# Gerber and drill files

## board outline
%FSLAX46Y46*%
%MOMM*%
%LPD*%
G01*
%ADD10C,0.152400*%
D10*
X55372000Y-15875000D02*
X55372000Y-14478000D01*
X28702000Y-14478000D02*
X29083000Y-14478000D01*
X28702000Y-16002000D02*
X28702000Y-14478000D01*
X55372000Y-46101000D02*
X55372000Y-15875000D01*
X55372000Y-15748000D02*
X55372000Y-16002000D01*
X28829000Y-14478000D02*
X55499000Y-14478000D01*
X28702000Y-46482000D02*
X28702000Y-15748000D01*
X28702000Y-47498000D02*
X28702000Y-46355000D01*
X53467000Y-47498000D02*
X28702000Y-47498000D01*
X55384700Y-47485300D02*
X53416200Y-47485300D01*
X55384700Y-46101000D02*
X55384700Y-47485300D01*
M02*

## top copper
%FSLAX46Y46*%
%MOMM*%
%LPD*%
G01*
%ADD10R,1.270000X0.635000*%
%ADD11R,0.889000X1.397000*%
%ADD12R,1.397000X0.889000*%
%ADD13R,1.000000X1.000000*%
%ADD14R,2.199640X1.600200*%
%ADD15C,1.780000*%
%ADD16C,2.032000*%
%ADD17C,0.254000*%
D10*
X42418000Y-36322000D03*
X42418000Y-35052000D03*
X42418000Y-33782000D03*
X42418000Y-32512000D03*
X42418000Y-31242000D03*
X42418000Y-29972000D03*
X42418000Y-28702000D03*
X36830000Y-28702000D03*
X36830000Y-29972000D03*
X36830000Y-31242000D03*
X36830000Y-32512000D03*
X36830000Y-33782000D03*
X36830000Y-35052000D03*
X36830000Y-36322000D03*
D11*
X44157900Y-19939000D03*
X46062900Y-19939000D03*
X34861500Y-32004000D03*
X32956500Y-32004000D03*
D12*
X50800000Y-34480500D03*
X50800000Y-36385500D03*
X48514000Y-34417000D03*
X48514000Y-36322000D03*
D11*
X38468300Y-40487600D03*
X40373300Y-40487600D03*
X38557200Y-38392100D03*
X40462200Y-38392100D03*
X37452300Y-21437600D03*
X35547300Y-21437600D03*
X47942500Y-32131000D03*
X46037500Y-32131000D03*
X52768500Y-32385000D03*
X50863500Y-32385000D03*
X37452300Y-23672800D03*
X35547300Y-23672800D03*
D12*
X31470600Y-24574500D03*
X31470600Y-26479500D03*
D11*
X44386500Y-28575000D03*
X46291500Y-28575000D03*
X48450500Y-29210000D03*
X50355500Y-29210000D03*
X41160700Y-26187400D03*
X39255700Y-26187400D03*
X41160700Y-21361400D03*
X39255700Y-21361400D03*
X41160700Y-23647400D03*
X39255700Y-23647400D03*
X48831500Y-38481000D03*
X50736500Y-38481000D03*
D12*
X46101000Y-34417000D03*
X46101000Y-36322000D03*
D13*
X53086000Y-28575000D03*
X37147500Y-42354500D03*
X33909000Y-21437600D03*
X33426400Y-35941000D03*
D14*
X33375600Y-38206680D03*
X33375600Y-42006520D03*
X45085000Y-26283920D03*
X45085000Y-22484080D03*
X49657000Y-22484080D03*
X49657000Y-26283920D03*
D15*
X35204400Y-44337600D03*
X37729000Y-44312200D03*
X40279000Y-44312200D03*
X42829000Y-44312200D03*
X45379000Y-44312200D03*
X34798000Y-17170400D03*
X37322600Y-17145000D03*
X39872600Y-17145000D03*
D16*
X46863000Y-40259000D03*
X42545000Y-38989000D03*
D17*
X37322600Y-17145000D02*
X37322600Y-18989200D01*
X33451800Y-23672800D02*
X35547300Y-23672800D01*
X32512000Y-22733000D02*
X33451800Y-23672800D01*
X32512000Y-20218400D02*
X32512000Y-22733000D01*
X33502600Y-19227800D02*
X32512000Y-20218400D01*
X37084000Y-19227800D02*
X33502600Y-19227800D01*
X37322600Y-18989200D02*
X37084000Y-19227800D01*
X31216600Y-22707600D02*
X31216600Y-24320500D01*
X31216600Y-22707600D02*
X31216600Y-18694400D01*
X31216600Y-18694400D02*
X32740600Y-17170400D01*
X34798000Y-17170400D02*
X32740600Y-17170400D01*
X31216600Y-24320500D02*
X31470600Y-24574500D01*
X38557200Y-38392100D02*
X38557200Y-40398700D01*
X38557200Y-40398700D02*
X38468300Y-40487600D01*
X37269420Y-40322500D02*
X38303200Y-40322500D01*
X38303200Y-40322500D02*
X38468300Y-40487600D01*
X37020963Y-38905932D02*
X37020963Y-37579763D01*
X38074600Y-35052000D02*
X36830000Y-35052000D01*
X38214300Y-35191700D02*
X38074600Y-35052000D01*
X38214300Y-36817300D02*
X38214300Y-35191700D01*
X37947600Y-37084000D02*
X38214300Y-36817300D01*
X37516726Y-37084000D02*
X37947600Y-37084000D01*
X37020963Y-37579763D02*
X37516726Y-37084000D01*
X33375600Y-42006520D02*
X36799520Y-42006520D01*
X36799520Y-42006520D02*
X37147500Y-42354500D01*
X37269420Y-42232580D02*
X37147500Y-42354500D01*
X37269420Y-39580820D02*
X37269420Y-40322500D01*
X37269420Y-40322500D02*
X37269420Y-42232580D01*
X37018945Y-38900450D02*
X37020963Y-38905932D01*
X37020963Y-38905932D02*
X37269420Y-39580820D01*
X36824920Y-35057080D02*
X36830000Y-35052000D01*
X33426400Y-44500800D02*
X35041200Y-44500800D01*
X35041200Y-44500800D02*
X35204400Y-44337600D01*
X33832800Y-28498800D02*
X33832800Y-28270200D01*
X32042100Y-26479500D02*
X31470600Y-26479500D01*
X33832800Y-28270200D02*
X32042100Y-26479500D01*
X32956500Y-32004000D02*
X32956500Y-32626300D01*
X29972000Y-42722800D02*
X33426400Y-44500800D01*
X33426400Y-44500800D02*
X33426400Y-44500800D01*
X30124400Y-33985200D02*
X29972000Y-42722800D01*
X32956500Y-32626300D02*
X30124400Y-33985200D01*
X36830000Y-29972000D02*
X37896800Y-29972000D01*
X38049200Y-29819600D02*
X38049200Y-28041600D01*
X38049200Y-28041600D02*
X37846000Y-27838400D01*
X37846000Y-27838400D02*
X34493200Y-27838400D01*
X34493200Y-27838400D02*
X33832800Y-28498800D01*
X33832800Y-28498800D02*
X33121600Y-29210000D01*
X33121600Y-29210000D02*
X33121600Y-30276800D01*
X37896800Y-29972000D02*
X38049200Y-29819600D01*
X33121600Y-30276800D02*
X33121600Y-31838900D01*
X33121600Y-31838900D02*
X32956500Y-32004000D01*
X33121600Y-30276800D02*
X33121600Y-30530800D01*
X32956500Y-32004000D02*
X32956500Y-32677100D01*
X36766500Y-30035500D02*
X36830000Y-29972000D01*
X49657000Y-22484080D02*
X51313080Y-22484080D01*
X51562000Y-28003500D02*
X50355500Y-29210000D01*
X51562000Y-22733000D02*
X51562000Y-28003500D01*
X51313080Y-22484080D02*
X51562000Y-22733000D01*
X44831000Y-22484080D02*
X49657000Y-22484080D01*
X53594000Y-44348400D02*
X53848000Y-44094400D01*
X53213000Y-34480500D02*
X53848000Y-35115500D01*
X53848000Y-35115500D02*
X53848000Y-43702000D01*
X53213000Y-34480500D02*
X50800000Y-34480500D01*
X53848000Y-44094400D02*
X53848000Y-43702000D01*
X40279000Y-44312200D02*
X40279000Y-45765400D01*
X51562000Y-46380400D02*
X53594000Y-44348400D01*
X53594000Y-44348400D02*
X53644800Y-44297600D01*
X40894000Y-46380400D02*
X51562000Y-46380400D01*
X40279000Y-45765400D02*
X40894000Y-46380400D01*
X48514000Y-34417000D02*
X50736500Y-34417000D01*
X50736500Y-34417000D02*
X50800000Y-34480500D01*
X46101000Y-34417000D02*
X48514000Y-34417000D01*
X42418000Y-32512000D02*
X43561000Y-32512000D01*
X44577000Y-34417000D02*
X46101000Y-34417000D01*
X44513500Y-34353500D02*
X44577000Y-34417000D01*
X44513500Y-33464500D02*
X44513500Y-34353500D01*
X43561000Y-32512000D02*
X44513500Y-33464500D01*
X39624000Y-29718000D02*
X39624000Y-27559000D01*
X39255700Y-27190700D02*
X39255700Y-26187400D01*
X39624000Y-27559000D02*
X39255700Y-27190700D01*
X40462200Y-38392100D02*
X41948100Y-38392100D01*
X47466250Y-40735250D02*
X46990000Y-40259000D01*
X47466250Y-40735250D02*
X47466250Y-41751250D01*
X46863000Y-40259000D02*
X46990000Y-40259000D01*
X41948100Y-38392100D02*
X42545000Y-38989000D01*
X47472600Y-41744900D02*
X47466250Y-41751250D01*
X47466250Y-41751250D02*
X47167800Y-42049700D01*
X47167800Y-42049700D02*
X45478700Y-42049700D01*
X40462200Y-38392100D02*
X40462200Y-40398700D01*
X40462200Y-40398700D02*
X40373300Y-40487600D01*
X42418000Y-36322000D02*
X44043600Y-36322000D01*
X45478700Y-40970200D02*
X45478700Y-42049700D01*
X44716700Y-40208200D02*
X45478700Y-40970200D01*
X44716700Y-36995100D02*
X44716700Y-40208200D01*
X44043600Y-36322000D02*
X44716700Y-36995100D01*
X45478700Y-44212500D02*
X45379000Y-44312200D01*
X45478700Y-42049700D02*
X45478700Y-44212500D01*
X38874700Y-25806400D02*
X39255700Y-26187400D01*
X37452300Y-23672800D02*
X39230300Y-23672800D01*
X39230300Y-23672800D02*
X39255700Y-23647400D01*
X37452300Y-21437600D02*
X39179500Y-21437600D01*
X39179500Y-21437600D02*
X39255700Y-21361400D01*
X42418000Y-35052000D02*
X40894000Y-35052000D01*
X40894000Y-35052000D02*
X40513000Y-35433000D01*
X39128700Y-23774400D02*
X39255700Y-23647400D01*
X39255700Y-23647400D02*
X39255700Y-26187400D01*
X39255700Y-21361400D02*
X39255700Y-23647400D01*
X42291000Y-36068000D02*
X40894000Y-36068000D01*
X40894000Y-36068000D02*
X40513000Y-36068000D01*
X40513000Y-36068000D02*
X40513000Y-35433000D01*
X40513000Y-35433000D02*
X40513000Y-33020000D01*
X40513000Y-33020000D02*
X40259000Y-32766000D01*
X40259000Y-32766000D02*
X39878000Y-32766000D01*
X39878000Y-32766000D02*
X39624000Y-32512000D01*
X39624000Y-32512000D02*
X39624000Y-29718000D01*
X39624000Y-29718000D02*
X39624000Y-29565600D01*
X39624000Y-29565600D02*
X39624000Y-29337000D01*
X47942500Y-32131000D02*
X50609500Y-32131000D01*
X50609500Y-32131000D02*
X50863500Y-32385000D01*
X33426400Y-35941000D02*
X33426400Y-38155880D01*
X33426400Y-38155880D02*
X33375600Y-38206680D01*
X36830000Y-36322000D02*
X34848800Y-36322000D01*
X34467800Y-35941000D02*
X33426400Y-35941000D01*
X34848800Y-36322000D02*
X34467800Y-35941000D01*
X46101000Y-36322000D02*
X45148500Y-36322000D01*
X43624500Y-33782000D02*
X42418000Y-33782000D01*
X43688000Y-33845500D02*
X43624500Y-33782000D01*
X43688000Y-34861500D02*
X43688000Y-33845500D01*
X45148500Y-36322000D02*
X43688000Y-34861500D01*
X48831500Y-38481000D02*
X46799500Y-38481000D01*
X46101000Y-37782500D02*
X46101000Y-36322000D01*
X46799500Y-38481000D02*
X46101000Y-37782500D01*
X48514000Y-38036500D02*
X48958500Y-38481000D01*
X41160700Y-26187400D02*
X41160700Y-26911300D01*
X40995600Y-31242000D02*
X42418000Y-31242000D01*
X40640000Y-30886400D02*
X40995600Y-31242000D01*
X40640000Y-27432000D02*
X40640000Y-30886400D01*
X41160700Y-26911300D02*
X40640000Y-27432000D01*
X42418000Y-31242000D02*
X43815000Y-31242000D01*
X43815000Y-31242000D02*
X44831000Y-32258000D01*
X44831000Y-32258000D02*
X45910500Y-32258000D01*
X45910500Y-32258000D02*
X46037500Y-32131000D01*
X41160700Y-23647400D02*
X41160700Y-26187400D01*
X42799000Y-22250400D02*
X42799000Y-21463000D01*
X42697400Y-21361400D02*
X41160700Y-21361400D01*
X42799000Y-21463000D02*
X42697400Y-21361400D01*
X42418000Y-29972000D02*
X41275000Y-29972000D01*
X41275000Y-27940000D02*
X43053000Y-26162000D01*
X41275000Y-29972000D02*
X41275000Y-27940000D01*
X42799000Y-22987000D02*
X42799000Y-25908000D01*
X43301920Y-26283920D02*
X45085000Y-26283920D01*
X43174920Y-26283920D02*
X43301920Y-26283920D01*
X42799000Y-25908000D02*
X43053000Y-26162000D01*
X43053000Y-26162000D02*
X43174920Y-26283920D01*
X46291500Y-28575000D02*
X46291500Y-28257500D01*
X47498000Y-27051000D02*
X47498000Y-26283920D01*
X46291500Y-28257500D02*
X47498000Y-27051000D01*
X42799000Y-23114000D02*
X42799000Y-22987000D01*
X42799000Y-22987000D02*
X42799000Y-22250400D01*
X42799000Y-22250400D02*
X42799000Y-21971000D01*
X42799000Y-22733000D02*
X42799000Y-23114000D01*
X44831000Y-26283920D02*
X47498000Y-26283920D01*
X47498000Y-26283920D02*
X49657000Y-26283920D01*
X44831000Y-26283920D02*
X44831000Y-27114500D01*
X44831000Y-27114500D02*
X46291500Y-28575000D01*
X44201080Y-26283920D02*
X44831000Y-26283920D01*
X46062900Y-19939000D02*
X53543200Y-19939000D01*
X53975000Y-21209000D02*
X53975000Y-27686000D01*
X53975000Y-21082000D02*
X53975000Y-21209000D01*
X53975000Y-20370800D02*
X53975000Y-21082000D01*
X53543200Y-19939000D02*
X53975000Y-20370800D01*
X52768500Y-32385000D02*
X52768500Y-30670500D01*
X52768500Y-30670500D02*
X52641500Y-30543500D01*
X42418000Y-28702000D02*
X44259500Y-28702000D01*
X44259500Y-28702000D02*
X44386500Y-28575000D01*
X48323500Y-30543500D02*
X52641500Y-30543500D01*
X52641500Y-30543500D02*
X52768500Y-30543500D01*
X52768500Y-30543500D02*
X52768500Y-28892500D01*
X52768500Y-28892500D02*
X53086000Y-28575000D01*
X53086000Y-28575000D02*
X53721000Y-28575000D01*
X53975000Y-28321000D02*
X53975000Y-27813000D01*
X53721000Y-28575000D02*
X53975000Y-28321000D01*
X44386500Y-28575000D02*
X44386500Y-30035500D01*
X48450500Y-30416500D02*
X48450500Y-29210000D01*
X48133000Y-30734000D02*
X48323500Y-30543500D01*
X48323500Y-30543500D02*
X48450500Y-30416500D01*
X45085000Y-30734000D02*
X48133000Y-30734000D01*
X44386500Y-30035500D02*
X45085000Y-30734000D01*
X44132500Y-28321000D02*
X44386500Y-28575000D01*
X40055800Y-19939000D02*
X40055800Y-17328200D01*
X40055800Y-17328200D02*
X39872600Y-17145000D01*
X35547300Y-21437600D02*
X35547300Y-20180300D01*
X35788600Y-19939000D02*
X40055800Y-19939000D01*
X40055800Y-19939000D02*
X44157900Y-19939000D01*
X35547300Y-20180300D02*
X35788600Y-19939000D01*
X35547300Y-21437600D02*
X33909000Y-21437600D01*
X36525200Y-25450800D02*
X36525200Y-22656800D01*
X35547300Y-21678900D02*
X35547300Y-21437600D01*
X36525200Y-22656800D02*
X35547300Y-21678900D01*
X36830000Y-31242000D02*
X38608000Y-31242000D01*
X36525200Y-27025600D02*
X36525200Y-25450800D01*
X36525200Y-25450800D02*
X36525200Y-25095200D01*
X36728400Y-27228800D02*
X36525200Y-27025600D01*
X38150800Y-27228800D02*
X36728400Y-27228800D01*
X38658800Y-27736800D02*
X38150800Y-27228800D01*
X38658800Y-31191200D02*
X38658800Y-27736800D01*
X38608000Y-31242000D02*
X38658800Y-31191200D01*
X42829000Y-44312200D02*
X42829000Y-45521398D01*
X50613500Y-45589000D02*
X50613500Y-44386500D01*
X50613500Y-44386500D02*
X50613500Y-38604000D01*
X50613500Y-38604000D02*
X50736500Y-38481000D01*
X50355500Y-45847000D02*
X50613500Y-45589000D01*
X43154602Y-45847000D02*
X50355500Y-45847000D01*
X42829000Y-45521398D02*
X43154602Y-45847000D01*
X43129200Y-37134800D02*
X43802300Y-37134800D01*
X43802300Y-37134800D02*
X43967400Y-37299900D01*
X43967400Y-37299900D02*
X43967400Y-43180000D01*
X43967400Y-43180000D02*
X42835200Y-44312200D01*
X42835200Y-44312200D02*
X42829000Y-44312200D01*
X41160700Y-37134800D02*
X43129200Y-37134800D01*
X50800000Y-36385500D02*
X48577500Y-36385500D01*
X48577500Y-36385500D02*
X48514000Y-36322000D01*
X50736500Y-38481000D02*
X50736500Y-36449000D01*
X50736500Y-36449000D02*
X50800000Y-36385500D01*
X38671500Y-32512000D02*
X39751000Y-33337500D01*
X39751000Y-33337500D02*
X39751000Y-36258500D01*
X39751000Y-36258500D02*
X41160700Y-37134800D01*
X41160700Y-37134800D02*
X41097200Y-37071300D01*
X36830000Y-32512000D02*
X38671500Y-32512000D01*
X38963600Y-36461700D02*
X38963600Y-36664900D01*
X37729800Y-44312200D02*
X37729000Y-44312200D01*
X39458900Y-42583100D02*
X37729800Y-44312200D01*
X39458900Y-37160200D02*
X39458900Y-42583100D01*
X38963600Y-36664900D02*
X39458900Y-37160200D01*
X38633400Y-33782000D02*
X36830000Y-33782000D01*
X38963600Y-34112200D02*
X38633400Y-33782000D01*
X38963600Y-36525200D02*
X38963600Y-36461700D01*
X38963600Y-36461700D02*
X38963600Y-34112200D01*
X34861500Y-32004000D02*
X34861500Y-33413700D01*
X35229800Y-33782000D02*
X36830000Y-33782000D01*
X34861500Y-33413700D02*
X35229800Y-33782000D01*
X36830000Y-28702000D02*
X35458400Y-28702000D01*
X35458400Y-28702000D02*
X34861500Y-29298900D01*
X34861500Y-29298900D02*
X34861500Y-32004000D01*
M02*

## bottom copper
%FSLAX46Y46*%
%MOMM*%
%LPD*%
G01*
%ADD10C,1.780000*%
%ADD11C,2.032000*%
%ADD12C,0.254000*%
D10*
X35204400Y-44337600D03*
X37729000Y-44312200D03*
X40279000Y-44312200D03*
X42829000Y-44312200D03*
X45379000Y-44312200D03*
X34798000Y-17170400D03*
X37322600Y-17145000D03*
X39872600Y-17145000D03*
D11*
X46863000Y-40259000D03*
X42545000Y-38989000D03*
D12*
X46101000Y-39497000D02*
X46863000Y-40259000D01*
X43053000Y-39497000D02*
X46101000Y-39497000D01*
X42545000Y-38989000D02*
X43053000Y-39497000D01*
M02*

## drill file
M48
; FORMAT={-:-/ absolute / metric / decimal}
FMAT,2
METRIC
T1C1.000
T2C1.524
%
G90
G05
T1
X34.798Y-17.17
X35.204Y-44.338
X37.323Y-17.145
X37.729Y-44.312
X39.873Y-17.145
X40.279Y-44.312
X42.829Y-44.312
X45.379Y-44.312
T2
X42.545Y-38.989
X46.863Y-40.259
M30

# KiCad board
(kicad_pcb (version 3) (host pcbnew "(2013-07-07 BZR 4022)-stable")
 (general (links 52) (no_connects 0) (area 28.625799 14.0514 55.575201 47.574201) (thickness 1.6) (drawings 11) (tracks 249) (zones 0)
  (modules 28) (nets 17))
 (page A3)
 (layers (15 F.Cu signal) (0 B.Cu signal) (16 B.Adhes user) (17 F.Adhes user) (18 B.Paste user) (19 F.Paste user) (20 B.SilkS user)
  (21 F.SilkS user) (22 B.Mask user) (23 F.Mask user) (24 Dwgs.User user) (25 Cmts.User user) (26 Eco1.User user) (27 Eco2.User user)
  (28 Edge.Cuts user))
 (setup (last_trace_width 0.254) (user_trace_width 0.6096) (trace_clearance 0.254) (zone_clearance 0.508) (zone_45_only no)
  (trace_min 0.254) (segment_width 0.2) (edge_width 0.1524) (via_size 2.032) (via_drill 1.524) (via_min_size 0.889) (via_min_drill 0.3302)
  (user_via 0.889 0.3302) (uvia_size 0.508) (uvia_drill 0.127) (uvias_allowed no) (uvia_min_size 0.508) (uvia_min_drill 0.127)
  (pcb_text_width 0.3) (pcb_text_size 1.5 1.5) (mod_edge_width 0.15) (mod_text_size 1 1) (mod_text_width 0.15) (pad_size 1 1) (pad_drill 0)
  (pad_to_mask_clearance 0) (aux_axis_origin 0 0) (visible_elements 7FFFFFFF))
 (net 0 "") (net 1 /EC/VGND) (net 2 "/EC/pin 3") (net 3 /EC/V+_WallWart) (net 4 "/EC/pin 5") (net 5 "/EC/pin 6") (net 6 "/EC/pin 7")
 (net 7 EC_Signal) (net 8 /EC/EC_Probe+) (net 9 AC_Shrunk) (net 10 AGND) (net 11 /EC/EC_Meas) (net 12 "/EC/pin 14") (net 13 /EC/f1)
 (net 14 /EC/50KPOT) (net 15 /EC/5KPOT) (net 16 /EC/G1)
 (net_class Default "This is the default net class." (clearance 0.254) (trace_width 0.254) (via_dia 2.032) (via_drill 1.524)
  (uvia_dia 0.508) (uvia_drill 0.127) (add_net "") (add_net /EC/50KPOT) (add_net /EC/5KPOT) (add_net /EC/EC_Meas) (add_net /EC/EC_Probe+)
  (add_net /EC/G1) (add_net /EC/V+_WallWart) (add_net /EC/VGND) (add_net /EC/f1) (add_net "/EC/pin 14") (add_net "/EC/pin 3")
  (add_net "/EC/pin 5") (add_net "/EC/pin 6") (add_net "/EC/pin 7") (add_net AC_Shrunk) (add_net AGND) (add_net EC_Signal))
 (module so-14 (layer F.Cu) (at 39.624 32.512 90)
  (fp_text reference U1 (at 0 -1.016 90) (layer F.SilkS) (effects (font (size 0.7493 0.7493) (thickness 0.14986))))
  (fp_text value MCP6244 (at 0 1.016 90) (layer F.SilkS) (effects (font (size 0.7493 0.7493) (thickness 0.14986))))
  (pad 1 smd rect (at -3.81 2.794 90) (size 0.635 1.27) (layers F.Cu F.Paste F.Mask) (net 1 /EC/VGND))
  (pad 2 smd rect (at -2.54 2.794 90) (size 0.635 1.27) (layers F.Cu F.Paste F.Mask) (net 1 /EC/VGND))
  (pad 3 smd rect (at -1.27 2.794 90) (size 0.635 1.27) (layers F.Cu F.Paste F.Mask) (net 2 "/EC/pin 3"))
  (pad 4 smd rect (at 0 2.794 90) (size 0.635 1.27) (layers F.Cu F.Paste F.Mask) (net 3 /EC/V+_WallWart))
  (pad 5 smd rect (at 1.27 2.794 90) (size 0.635 1.27) (layers F.Cu F.Paste F.Mask) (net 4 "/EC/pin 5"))
  (pad 6 smd rect (at 2.54 2.794 90) (size 0.635 1.27) (layers F.Cu F.Paste F.Mask) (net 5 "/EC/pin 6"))
  (pad 7 smd rect (at 3.81 2.794 90) (size 0.635 1.27) (layers F.Cu F.Paste F.Mask) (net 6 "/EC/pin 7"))
  (pad 8 smd rect (at 3.81 -2.794 90) (size 0.635 1.27) (layers F.Cu F.Paste F.Mask) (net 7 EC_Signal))
  (pad 9 smd rect (at 2.54 -2.794 90) (size 0.635 1.27) (layers F.Cu F.Paste F.Mask) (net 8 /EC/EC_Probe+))
  (pad 10 smd rect (at 1.27 -2.794 90) (size 0.635 1.27) (layers F.Cu F.Paste F.Mask) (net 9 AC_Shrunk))
  (pad 11 smd rect (at 0 -2.794 90) (size 0.635 1.27) (layers F.Cu F.Paste F.Mask) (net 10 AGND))
  (pad 12 smd rect (at -1.27 -2.794 90) (size 0.635 1.27) (layers F.Cu F.Paste F.Mask) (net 7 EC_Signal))
  (pad 13 smd rect (at -2.54 -2.794 90) (size 0.635 1.27) (layers F.Cu F.Paste F.Mask) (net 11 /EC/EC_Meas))
  (pad 14 smd rect (at -3.81 -2.794 90) (size 0.635 1.27) (layers F.Cu F.Paste F.Mask) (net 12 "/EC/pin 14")))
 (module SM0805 (layer F.Cu) (at 45.1104 19.939)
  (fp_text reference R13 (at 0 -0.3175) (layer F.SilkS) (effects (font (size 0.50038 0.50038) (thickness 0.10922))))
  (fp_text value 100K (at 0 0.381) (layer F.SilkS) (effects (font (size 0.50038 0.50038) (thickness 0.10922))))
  (pad 1 smd rect (at -0.9525 0) (size 0.889 1.397) (layers F.Cu F.Paste F.Mask) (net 9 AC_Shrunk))
  (pad 2 smd rect (at 0.9525 0) (size 0.889 1.397) (layers F.Cu F.Paste F.Mask) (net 6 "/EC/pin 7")))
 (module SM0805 (layer F.Cu) (at 33.909 32.004 180)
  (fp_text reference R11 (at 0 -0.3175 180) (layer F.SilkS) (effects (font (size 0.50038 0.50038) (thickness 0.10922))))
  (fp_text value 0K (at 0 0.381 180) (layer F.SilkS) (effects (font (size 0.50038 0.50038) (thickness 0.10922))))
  (pad 1 smd rect (at -0.9525 0 180) (size 0.889 1.397) (layers F.Cu F.Paste F.Mask) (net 7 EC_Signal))
  (pad 2 smd rect (at 0.9525 0 180) (size 0.889 1.397) (layers F.Cu F.Paste F.Mask) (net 8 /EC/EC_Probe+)))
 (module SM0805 (layer F.Cu) (at 50.8 35.433 270)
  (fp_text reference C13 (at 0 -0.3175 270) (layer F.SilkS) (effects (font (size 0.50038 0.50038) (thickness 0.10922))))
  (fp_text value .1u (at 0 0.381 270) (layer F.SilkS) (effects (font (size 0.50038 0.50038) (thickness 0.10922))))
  (pad 1 smd rect (at -0.9525 0 270) (size 0.889 1.397) (layers F.Cu F.Paste F.Mask) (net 3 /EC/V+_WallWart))
  (pad 2 smd rect (at 0.9525 0 270) (size 0.889 1.397) (layers F.Cu F.Paste F.Mask) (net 10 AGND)))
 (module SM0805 (layer F.Cu) (at 48.514 35.3695 270)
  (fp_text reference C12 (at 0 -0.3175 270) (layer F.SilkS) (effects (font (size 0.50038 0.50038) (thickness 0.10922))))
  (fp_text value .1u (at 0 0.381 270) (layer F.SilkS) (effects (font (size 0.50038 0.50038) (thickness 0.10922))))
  (pad 1 smd rect (at -0.9525 0 270) (size 0.889 1.397) (layers F.Cu F.Paste F.Mask) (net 3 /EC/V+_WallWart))
  (pad 2 smd rect (at 0.9525 0 270) (size 0.889 1.397) (layers F.Cu F.Paste F.Mask) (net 10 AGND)))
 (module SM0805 (layer F.Cu) (at 39.4208 40.4876)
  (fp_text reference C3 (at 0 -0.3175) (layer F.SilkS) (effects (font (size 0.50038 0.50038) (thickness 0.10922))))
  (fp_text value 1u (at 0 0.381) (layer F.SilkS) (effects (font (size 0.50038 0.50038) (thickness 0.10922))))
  (pad 1 smd rect (at -0.9525 0) (size 0.889 1.397) (layers F.Cu F.Paste F.Mask) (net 11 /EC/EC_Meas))
  (pad 2 smd rect (at 0.9525 0) (size 0.889 1.397) (layers F.Cu F.Paste F.Mask) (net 1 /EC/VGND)))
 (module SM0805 (layer F.Cu) (at 39.5097 38.3921)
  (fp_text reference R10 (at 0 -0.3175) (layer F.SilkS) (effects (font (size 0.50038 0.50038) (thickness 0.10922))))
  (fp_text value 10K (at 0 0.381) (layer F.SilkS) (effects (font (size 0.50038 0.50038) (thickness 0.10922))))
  (pad 1 smd rect (at -0.9525 0) (size 0.889 1.397) (layers F.Cu F.Paste F.Mask) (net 11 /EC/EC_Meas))
  (pad 2 smd rect (at 0.9525 0) (size 0.889 1.397) (layers F.Cu F.Paste F.Mask) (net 1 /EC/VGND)))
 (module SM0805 (layer F.Cu) (at 36.4998 21.4376 180)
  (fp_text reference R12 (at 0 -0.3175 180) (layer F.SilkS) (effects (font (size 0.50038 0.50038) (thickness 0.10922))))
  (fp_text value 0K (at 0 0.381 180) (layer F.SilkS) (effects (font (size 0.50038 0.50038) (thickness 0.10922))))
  (pad 1 smd rect (at -0.9525 0 180) (size 0.889 1.397) (layers F.Cu F.Paste F.Mask) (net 1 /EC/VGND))
  (pad 2 smd rect (at 0.9525 0 180) (size 0.889 1.397) (layers F.Cu F.Paste F.Mask) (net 9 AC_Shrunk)))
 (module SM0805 (layer F.Cu) (at 46.99 32.131 180)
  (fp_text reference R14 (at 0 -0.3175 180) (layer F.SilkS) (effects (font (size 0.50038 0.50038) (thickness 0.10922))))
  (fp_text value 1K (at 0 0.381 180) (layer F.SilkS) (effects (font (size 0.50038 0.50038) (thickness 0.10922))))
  (pad 1 smd rect (at -0.9525 0 180) (size 0.889 1.397) (layers F.Cu F.Paste F.Mask) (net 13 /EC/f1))
  (pad 2 smd rect (at 0.9525 0 180) (size 0.889 1.397) (layers F.Cu F.Paste F.Mask) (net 4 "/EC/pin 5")))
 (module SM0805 (layer F.Cu) (at 51.816 32.385 180)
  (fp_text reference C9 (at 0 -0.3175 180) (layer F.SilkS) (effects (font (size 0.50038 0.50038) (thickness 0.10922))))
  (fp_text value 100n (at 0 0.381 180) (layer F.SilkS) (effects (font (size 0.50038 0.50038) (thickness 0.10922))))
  (pad 1 smd rect (at -0.9525 0 180) (size 0.889 1.397) (layers F.Cu F.Paste F.Mask) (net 6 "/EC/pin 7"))
  (pad 2 smd rect (at 0.9525 0 180) (size 0.889 1.397) (layers F.Cu F.Paste F.Mask) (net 13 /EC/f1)))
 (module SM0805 (layer F.Cu) (at 36.4998 23.6728 180)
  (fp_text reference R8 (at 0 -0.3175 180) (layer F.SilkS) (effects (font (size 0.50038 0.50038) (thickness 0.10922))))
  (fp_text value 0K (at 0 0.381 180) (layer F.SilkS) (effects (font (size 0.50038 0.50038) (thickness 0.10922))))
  (pad 1 smd rect (at -0.9525 0 180) (size 0.889 1.397) (layers F.Cu F.Paste F.Mask) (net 1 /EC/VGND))
  (pad 2 smd rect (at 0.9525 0 180) (size 0.889 1.397) (layers F.Cu F.Paste F.Mask) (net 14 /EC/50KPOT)))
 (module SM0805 (layer F.Cu) (at 31.4706 25.527 270)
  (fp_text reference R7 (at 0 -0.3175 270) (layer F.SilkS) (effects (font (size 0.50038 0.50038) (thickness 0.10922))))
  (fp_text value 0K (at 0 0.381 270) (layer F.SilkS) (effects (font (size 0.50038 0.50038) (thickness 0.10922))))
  (pad 1 smd rect (at -0.9525 0 270) (size 0.889 1.397) (layers F.Cu F.Paste F.Mask) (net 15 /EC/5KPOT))
  (pad 2 smd rect (at 0.9525 0 270) (size 0.889 1.397) (layers F.Cu F.Paste F.Mask) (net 8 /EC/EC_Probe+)))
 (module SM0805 (layer F.Cu) (at 45.339 28.575)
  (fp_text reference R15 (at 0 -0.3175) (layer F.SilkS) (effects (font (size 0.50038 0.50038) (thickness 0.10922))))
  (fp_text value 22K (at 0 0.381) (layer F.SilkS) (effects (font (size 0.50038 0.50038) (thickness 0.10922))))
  (pad 1 smd rect (at -0.9525 0) (size 0.889 1.397) (layers F.Cu F.Paste F.Mask) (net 6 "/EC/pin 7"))
  (pad 2 smd rect (at 0.9525 0) (size 0.889 1.397) (layers F.Cu F.Paste F.Mask) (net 5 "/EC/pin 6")))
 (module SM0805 (layer F.Cu) (at 49.403 29.21)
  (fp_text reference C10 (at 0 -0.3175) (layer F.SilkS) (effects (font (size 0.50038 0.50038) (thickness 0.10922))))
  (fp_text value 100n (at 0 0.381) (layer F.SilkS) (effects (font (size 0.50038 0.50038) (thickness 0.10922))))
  (pad 1 smd rect (at -0.9525 0) (size 0.889 1.397) (layers F.Cu F.Paste F.Mask) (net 6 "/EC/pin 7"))
  (pad 2 smd rect (at 0.9525 0) (size 0.889 1.397) (layers F.Cu F.Paste F.Mask) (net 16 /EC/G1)))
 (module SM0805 (layer F.Cu) (at 40.2082 26.1874 180)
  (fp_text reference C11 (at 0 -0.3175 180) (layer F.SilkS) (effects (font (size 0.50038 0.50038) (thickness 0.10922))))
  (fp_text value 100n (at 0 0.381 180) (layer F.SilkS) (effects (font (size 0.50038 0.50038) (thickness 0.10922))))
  (pad 1 smd rect (at -0.9525 0 180) (size 0.889 1.397) (layers F.Cu F.Paste F.Mask) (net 4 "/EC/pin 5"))
  (pad 2 smd rect (at 0.9525 0 180) (size 0.889 1.397) (layers F.Cu F.Paste F.Mask) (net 1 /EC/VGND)))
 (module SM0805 (layer F.Cu) (at 40.2082 21.3614 180)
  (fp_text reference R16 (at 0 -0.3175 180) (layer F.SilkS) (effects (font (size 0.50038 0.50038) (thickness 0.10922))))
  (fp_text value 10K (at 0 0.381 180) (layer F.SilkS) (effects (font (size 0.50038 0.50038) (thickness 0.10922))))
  (pad 1 smd rect (at -0.9525 0 180) (size 0.889 1.397) (layers F.Cu F.Paste F.Mask) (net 5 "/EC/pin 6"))
  (pad 2 smd rect (at 0.9525 0 180) (size 0.889 1.397) (layers F.Cu F.Paste F.Mask) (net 1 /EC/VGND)))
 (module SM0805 (layer F.Cu) (at 40.2082 23.6474 180)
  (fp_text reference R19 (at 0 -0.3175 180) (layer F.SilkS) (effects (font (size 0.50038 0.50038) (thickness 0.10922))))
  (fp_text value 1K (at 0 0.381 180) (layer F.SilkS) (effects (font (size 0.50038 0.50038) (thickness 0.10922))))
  (pad 1 smd rect (at -0.9525 0 180) (size 0.889 1.397) (layers F.Cu F.Paste F.Mask) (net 4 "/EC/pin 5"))
  (pad 2 smd rect (at 0.9525 0 180) (size 0.889 1.397) (layers F.Cu F.Paste F.Mask) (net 1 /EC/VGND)))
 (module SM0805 (layer F.Cu) (at 49.784 38.481)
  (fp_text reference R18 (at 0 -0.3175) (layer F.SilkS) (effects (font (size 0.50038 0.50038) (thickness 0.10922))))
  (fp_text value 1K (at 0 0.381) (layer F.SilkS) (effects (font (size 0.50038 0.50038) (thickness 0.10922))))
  (pad 1 smd rect (at -0.9525 0) (size 0.889 1.397) (layers F.Cu F.Paste F.Mask) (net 2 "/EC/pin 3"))
  (pad 2 smd rect (at 0.9525 0) (size 0.889 1.397) (layers F.Cu F.Paste F.Mask) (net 10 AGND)))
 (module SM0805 (layer F.Cu) (at 46.101 35.3695 270)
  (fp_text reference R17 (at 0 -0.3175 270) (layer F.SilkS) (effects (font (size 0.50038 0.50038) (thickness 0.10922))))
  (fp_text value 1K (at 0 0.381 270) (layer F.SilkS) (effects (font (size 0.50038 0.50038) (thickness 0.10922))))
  (pad 1 smd rect (at -0.9525 0 270) (size 0.889 1.397) (layers F.Cu F.Paste F.Mask) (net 3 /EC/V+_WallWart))
  (pad 2 smd rect (at 0.9525 0 270) (size 0.889 1.397) (layers F.Cu F.Paste F.Mask) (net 2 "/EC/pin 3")))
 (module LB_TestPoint (layer F.Cu) (at 53.086 28.575)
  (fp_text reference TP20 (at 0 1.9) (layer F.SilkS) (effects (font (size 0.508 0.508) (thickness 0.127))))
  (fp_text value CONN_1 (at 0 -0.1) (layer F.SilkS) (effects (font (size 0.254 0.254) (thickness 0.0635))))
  (pad 1 smd rect (at 0 0) (size 1 1) (layers F.Cu F.Paste F.Mask) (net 6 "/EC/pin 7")))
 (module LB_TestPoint (layer F.Cu) (at 37.1475 42.3545 90)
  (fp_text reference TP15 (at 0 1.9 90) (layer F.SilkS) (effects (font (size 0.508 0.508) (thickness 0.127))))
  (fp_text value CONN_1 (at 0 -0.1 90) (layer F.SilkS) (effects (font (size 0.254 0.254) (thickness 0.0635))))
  (pad 1 smd rect (at 0 0 90) (size 1 1) (layers F.Cu F.Paste F.Mask) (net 11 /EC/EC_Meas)))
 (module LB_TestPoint (layer F.Cu) (at 33.909 21.4376)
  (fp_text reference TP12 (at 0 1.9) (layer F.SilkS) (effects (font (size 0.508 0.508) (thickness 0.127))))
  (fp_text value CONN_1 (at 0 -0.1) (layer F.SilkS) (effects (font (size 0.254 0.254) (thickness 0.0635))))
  (pad 1 smd rect (at 0 0) (size 1 1) (layers F.Cu F.Paste F.Mask) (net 9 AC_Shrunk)))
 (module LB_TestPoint (layer F.Cu) (at 33.4264 35.941)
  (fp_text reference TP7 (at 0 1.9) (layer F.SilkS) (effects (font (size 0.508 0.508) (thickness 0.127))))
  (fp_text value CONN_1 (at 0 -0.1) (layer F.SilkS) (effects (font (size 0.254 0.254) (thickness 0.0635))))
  (pad 1 smd rect (at 0 0) (size 1 1) (layers F.Cu F.Paste F.Mask) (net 12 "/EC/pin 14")))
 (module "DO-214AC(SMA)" (layer F.Cu) (at 33.3756 40.1066 270)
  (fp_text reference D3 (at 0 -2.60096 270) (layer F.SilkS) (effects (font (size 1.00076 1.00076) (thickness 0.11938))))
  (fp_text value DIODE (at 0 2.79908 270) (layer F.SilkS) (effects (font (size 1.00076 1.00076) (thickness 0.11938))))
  (pad 1 smd rect (at -1.89992 0 270) (size 1.6002 2.19964) (layers F.Cu F.Paste F.Mask) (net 12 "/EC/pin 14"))
  (pad 2 smd rect (at 1.89992 0 270) (size 1.6002 2.19964) (layers F.Cu F.Paste F.Mask) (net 11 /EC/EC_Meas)))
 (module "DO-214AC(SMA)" (layer F.Cu) (at 45.085 24.384 90)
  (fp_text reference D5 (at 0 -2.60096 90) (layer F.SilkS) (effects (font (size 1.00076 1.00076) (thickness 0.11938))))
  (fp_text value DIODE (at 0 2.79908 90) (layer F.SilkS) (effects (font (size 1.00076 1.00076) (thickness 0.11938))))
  (pad 1 smd rect (at -1.89992 0 90) (size 1.6002 2.19964) (layers F.Cu F.Paste F.Mask) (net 5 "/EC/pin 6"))
  (pad 2 smd rect (at 1.89992 0 90) (size 1.6002 2.19964) (layers F.Cu F.Paste F.Mask) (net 16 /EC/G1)))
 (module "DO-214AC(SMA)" (layer F.Cu) (at 49.657 24.384 270)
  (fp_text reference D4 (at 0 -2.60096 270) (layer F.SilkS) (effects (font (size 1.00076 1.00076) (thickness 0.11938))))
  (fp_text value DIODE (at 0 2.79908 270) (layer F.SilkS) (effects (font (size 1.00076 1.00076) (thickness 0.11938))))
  (pad 1 smd rect (at -1.89992 0 270) (size 1.6002 2.19964) (layers F.Cu F.Paste F.Mask) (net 16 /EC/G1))
  (pad 2 smd rect (at 1.89992 0 270) (size 1.6002 2.19964) (layers F.Cu F.Paste F.Mask) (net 5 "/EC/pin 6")))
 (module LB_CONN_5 (layer F.Cu) (at 35.2044 44.2976)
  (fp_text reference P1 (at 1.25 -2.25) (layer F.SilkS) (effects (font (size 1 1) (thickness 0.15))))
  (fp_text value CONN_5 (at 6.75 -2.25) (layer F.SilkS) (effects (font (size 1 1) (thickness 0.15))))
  (pad 1 thru_hole circle (at 0 0.04) (size 1.78 1.78) (drill 1) (layers *.Cu *.Mask F.SilkS) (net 8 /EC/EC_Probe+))
  (pad 2 thru_hole circle (at 2.5246 0.0146) (size 1.78 1.78) (drill 1) (layers *.Cu *.Mask F.SilkS) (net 7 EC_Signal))
  (pad 3 thru_hole circle (at 5.0746 0.0146) (size 1.78 1.78) (drill 1) (layers *.Cu *.Mask F.SilkS) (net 3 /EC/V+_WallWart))
  (pad 4 thru_hole circle (at 7.6246 0.0146) (size 1.78 1.78) (drill 1) (layers *.Cu *.Mask F.SilkS) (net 10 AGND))
  (pad 5 thru_hole circle (at 10.1746 0.0146) (size 1.78 1.78) (drill 1) (layers *.Cu *.Mask F.SilkS) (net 1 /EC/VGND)))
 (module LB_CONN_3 (layer F.Cu) (at 34.798 14.6304)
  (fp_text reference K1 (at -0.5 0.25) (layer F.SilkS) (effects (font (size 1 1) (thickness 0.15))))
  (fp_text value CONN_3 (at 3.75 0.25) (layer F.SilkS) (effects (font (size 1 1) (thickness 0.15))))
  (pad 1 thru_hole circle (at 0 2.54) (size 1.78 1.78) (drill 1) (layers *.Cu *.Mask F.SilkS) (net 15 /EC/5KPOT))
  (pad 2 thru_hole circle (at 2.5246 2.5146) (size 1.78 1.78) (drill 1) (layers *.Cu *.Mask F.SilkS) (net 14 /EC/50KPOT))
  (pad 3 thru_hole circle (at 5.0746 2.5146) (size 1.78 1.78) (drill 1) (layers *.Cu *.Mask F.SilkS) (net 9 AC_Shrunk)))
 (gr_line (start 55.372 15.875) (end 55.372 14.478) (angle 90) (layer Edge.Cuts) (width 0.1524))
 (gr_line (start 28.702 14.478) (end 29.083 14.478) (angle 90) (layer Edge.Cuts) (width 0.1524))
 (gr_line (start 28.702 16.002) (end 28.702 14.478) (angle 90) (layer Edge.Cuts) (width 0.1524))
 (gr_line (start 55.372 46.101) (end 55.372 15.875) (angle 90) (layer Edge.Cuts) (width 0.1524))
 (gr_line (start 55.372 15.748) (end 55.372 16.002) (angle 90) (layer Edge.Cuts) (width 0.1524))
 (gr_line (start 28.829 14.478) (end 55.499 14.478) (angle 90) (layer Edge.Cuts) (width 0.1524))
 (gr_line (start 28.702 46.482) (end 28.702 15.748) (angle 90) (layer Edge.Cuts) (width 0.1524))
 (gr_line (start 28.702 47.498) (end 28.702 46.355) (angle 90) (layer Edge.Cuts) (width 0.1524))
 (gr_line (start 53.467 47.498) (end 28.702 47.498) (angle 90) (layer Edge.Cuts) (width 0.1524))
 (gr_line (start 55.3847 47.4853) (end 53.4162 47.4853) (angle 90) (layer Edge.Cuts) (width 0.1524))
 (gr_line (start 55.3847 46.101) (end 55.3847 47.4853) (angle 90) (layer Edge.Cuts) (width 0.1524))
 (segment (start 37.3226 17.145) (end 37.3226 18.9892) (width 0.254) (layer F.Cu) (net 14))
 (segment (start 33.4518 23.6728) (end 35.5473 23.6728) (width 0.254) (layer F.Cu) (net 14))
 (segment (start 32.512 22.733) (end 33.4518 23.6728) (width 0.254) (layer F.Cu) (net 14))
 (segment (start 32.512 20.2184) (end 32.512 22.733) (width 0.254) (layer F.Cu) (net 14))
 (segment (start 33.5026 19.2278) (end 32.512 20.2184) (width 0.254) (layer F.Cu) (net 14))
 (segment (start 37.084 19.2278) (end 33.5026 19.2278) (width 0.254) (layer F.Cu) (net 14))
 (segment (start 37.3226 18.9892) (end 37.084 19.2278) (width 0.254) (layer F.Cu) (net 14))
 (segment (start 31.2166 22.7076) (end 31.2166 24.3205) (width 0.254) (layer F.Cu) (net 15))
 (segment (start 31.2166 22.7076) (end 31.2166 18.6944) (width 0.254) (layer F.Cu) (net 15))
 (segment (start 31.2166 18.6944) (end 32.7406 17.1704) (width 0.254) (layer F.Cu) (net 15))
 (segment (start 34.798 17.1704) (end 32.7406 17.1704) (width 0.254) (layer F.Cu) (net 15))
 (segment (start 31.2166 24.3205) (end 31.4706 24.5745) (width 0.254) (layer F.Cu) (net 15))
 (segment (start 38.5572 38.3921) (end 38.5572 40.3987) (width 0.254) (layer F.Cu) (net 11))
 (segment (start 38.5572 40.3987) (end 38.4683 40.4876) (width 0.254) (layer F.Cu) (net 11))
 (segment (start 37.26942 40.3225) (end 38.3032 40.3225) (width 0.254) (layer F.Cu) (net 11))
 (segment (start 38.3032 40.3225) (end 38.4683 40.4876) (width 0.254) (layer F.Cu) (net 11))
 (segment (start 37.020963 38.905932) (end 37.020963 37.579763) (width 0.254) (layer F.Cu) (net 11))
 (segment (start 38.0746 35.052) (end 36.83 35.052) (width 0.254) (layer F.Cu) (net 11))
 (segment (start 38.2143 35.1917) (end 38.0746 35.052) (width 0.254) (layer F.Cu) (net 11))
 (segment (start 38.2143 36.8173) (end 38.2143 35.1917) (width 0.254) (layer F.Cu) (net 11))
 (segment (start 37.9476 37.084) (end 38.2143 36.8173) (width 0.254) (layer F.Cu) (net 11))
 (segment (start 37.516726 37.084) (end 37.9476 37.084) (width 0.254) (layer F.Cu) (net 11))
 (segment (start 37.020963 37.579763) (end 37.516726 37.084) (width 0.254) (layer F.Cu) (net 11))
 (segment (start 33.3756 42.00652) (end 36.79952 42.00652) (width 0.254) (layer F.Cu) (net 11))
 (segment (start 36.79952 42.00652) (end 37.1475 42.3545) (width 0.254) (layer F.Cu) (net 11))
 (segment (start 37.26942 42.23258) (end 37.1475 42.3545) (width 0.254) (layer F.Cu) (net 11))
 (segment (start 37.26942 39.58082) (end 37.26942 40.3225) (width 0.254) (layer F.Cu) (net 11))
 (segment (start 37.26942 40.3225) (end 37.26942 42.23258) (width 0.254) (layer F.Cu) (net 11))
 (segment (start 37.018945 38.90045) (end 37.020963 38.905932) (width 0.254) (layer F.Cu) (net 11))
 (segment (start 37.020963 38.905932) (end 37.26942 39.58082) (width 0.254) (layer F.Cu) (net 11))
 (segment (start 36.82492 35.05708) (end 36.83 35.052) (width 0.254) (layer F.Cu) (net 11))
 (segment (start 33.4264 44.5008) (end 35.0412 44.5008) (width 0.254) (layer F.Cu) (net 8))
 (segment (start 35.0412 44.5008) (end 35.2044 44.3376) (width 0.254) (layer F.Cu) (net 8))
 (segment (start 33.8328 28.4988) (end 33.8328 28.2702) (width 0.254) (layer F.Cu) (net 8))
 (segment (start 32.0421 26.4795) (end 31.4706 26.4795) (width 0.254) (layer F.Cu) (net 8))
 (segment (start 33.8328 28.2702) (end 32.0421 26.4795) (width 0.254) (layer F.Cu) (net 8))
 (segment (start 32.9565 32.004) (end 32.9565 32.6263) (width 0.254) (layer F.Cu) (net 8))
 (segment (start 29.972 42.7228) (end 33.4264 44.5008) (width 0.254) (layer F.Cu) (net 8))
 (segment (start 33.4264 44.5008) (end 33.4264 44.5008) (width 0.254) (layer F.Cu) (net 8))
 (segment (start 30.1244 33.9852) (end 29.972 42.7228) (width 0.254) (layer F.Cu) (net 8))
 (segment (start 32.9565 32.6263) (end 30.1244 33.9852) (width 0.254) (layer F.Cu) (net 8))
 (segment (start 36.83 29.972) (end 37.8968 29.972) (width 0.254) (layer F.Cu) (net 8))
 (segment (start 38.0492 29.8196) (end 38.0492 28.0416) (width 0.254) (layer F.Cu) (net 8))
 (segment (start 38.0492 28.0416) (end 37.846 27.8384) (width 0.254) (layer F.Cu) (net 8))
 (segment (start 37.846 27.8384) (end 34.4932 27.8384) (width 0.254) (layer F.Cu) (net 8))
 (segment (start 34.4932 27.8384) (end 33.8328 28.4988) (width 0.254) (layer F.Cu) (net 8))
 (segment (start 33.8328 28.4988) (end 33.1216 29.21) (width 0.254) (layer F.Cu) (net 8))
 (segment (start 33.1216 29.21) (end 33.1216 30.2768) (width 0.254) (layer F.Cu) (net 8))
 (segment (start 37.8968 29.972) (end 38.0492 29.8196) (width 0.254) (layer F.Cu) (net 8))
 (segment (start 33.1216 30.2768) (end 33.1216 31.8389) (width 0.254) (layer F.Cu) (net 8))
 (segment (start 33.1216 31.8389) (end 32.9565 32.004) (width 0.254) (layer F.Cu) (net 8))
 (segment (start 33.1216 30.2768) (end 33.1216 30.5308) (width 0.254) (layer F.Cu) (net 8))
 (segment (start 32.9565 32.004) (end 32.9565 32.6771) (width 0.254) (layer F.Cu) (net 8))
 (segment (start 36.7665 30.0355) (end 36.83 29.972) (width 0.254) (layer F.Cu) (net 8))
 (segment (start 49.657 22.48408) (end 51.31308 22.48408) (width 0.254) (layer F.Cu) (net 16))
 (segment (start 51.562 28.0035) (end 50.3555 29.21) (width 0.254) (layer F.Cu) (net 16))
 (segment (start 51.562 22.733) (end 51.562 28.0035) (width 0.254) (layer F.Cu) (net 16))
 (segment (start 51.31308 22.48408) (end 51.562 22.733) (width 0.254) (layer F.Cu) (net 16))
 (segment (start 44.831 22.48408) (end 49.657 22.48408) (width 0.254) (layer F.Cu) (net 16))
 (segment (start 53.594 44.3484) (end 53.848 44.0944) (width 0.254) (layer F.Cu) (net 3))
 (segment (start 53.213 34.4805) (end 53.848 35.1155) (width 0.254) (layer F.Cu) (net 3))
 (segment (start 53.848 35.1155) (end 53.848 43.702) (width 0.254) (layer F.Cu) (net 3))
 (segment (start 53.213 34.4805) (end 50.8 34.4805) (width 0.254) (layer F.Cu) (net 3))
 (segment (start 53.848 44.0944) (end 53.848 43.702) (width 0.254) (layer F.Cu) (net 3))
 (segment (start 40.279 44.3122) (end 40.279 45.7654) (width 0.254) (layer F.Cu) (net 3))
 (segment (start 51.562 46.3804) (end 53.594 44.3484) (width 0.254) (layer F.Cu) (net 3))
 (segment (start 53.594 44.3484) (end 53.6448 44.2976) (width 0.254) (layer F.Cu) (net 3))
 (segment (start 40.894 46.3804) (end 51.562 46.3804) (width 0.254) (layer F.Cu) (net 3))
 (segment (start 40.279 45.7654) (end 40.894 46.3804) (width 0.254) (layer F.Cu) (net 3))
 (segment (start 48.514 34.417) (end 50.7365 34.417) (width 0.254) (layer F.Cu) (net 3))
 (segment (start 50.7365 34.417) (end 50.8 34.4805) (width 0.254) (layer F.Cu) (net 3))
 (segment (start 46.101 34.417) (end 48.514 34.417) (width 0.254) (layer F.Cu) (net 3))
 (segment (start 42.418 32.512) (end 43.561 32.512) (width 0.254) (layer F.Cu) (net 3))
 (segment (start 44.577 34.417) (end 46.101 34.417) (width 0.254) (layer F.Cu) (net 3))
 (segment (start 44.5135 34.3535) (end 44.577 34.417) (width 0.254) (layer F.Cu) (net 3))
 (segment (start 44.5135 33.4645) (end 44.5135 34.3535) (width 0.254) (layer F.Cu) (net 3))
 (segment (start 43.561 32.512) (end 44.5135 33.4645) (width 0.254) (layer F.Cu) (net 3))
 (segment (start 39.624 29.718) (end 39.624 27.559) (width 0.254) (layer F.Cu) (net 1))
 (segment (start 39.2557 27.1907) (end 39.2557 26.1874) (width 0.254) (layer F.Cu) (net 1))
 (segment (start 39.624 27.559) (end 39.2557 27.1907) (width 0.254) (layer F.Cu) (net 1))
 (segment (start 40.4622 38.3921) (end 41.9481 38.3921) (width 0.254) (layer F.Cu) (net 1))
 (segment (start 47.46625 40.73525) (end 46.99 40.259) (width 0.254) (layer F.Cu) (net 1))
 (segment (start 47.46625 40.73525) (end 47.46625 41.75125) (width 0.254) (layer F.Cu) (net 1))
 (segment (start 46.863 40.259) (end 46.99 40.259) (width 0.254) (layer F.Cu) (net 1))
 (via (at 46.863 40.259) (size 2.032) (layers F.Cu B.Cu) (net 1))
 (segment (start 46.101 39.497) (end 46.863 40.259) (width 0.254) (layer B.Cu) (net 1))
 (segment (start 43.053 39.497) (end 46.101 39.497) (width 0.254) (layer B.Cu) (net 1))
 (segment (start 42.545 38.989) (end 43.053 39.497) (width 0.254) (layer B.Cu) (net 1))
 (via (at 42.545 38.989) (size 2.032) (layers F.Cu B.Cu) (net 1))
 (segment (start 41.9481 38.3921) (end 42.545 38.989) (width 0.254) (layer F.Cu) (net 1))
 (segment (start 47.4726 41.7449) (end 47.46625 41.75125) (width 0.254) (layer F.Cu) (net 1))
 (segment (start 47.46625 41.75125) (end 47.1678 42.0497) (width 0.254) (layer F.Cu) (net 1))
 (segment (start 47.1678 42.0497) (end 45.4787 42.0497) (width 0.254) (layer F.Cu) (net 1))
 (segment (start 40.4622 38.3921) (end 40.4622 40.3987) (width 0.254) (layer F.Cu) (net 1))
 (segment (start 40.4622 40.3987) (end 40.3733 40.4876) (width 0.254) (layer F.Cu) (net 1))
 (segment (start 42.418 36.322) (end 44.0436 36.322) (width 0.254) (layer F.Cu) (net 1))
 (segment (start 45.4787 40.9702) (end 45.4787 42.0497) (width 0.254) (layer F.Cu) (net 1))
 (segment (start 44.7167 40.2082) (end 45.4787 40.9702) (width 0.254) (layer F.Cu) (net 1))
 (segment (start 44.7167 36.9951) (end 44.7167 40.2082) (width 0.254) (layer F.Cu) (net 1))
 (segment (start 44.0436 36.322) (end 44.7167 36.9951) (width 0.254) (layer F.Cu) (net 1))
 (segment (start 45.4787 44.2125) (end 45.379 44.3122) (width 0.254) (layer F.Cu) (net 1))
 (segment (start 45.4787 42.0497) (end 45.4787 44.2125) (width 0.254) (layer F.Cu) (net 1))
 (segment (start 38.8747 25.8064) (end 39.2557 26.1874) (width 0.254) (layer F.Cu) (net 1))
 (segment (start 37.4523 23.6728) (end 39.2303 23.6728) (width 0.254) (layer F.Cu) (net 1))
 (segment (start 39.2303 23.6728) (end 39.2557 23.6474) (width 0.254) (layer F.Cu) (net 1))
 (segment (start 37.4523 21.4376) (end 39.1795 21.4376) (width 0.254) (layer F.Cu) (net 1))
 (segment (start 39.1795 21.4376) (end 39.2557 21.3614) (width 0.254) (layer F.Cu) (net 1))
 (segment (start 42.418 35.052) (end 40.894 35.052) (width 0.254) (layer F.Cu) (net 1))
 (segment (start 40.894 35.052) (end 40.513 35.433) (width 0.254) (layer F.Cu) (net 1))
 (segment (start 39.1287 23.7744) (end 39.2557 23.6474) (width 0.254) (layer F.Cu) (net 1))
 (segment (start 39.2557 23.6474) (end 39.2557 26.1874) (width 0.254) (layer F.Cu) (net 1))
 (segment (start 39.2557 21.3614) (end 39.2557 23.6474) (width 0.254) (layer F.Cu) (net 1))
 (segment (start 42.291 36.068) (end 40.894 36.068) (width 0.254) (layer F.Cu) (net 1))
 (segment (start 40.894 36.068) (end 40.513 36.068) (width 0.254) (layer F.Cu) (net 1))
 (segment (start 40.513 36.068) (end 40.513 35.433) (width 0.254) (layer F.Cu) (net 1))
 (segment (start 40.513 35.433) (end 40.513 33.02) (width 0.254) (layer F.Cu) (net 1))
 (segment (start 40.513 33.02) (end 40.259 32.766) (width 0.254) (layer F.Cu) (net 1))
 (segment (start 40.259 32.766) (end 39.878 32.766) (width 0.254) (layer F.Cu) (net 1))
 (segment (start 39.878 32.766) (end 39.624 32.512) (width 0.254) (layer F.Cu) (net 1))
 (segment (start 39.624 32.512) (end 39.624 29.718) (width 0.254) (layer F.Cu) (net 1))
 (segment (start 39.624 29.718) (end 39.624 29.5656) (width 0.254) (layer F.Cu) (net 1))
 (segment (start 39.624 29.5656) (end 39.624 29.337) (width 0.254) (layer F.Cu) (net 1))
 (segment (start 47.9425 32.131) (end 50.6095 32.131) (width 0.254) (layer F.Cu) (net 13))
 (segment (start 50.6095 32.131) (end 50.8635 32.385) (width 0.254) (layer F.Cu) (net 13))
 (segment (start 33.4264 35.941) (end 33.4264 38.15588) (width 0.254) (layer F.Cu) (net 12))
 (segment (start 33.4264 38.15588) (end 33.3756 38.20668) (width 0.254) (layer F.Cu) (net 12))
 (segment (start 36.83 36.322) (end 34.8488 36.322) (width 0.254) (layer F.Cu) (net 12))
 (segment (start 34.4678 35.941) (end 33.4264 35.941) (width 0.254) (layer F.Cu) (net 12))
 (segment (start 34.8488 36.322) (end 34.4678 35.941) (width 0.254) (layer F.Cu) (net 12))
 (segment (start 46.101 36.322) (end 45.1485 36.322) (width 0.254) (layer F.Cu) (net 2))
 (segment (start 43.6245 33.782) (end 42.418 33.782) (width 0.254) (layer F.Cu) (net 2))
 (segment (start 43.688 33.8455) (end 43.6245 33.782) (width 0.254) (layer F.Cu) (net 2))
 (segment (start 43.688 34.8615) (end 43.688 33.8455) (width 0.254) (layer F.Cu) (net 2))
 (segment (start 45.1485 36.322) (end 43.688 34.8615) (width 0.254) (layer F.Cu) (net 2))
 (segment (start 48.8315 38.481) (end 46.7995 38.481) (width 0.254) (layer F.Cu) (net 2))
 (segment (start 46.101 37.7825) (end 46.101 36.322) (width 0.254) (layer F.Cu) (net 2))
 (segment (start 46.7995 38.481) (end 46.101 37.7825) (width 0.254) (layer F.Cu) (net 2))
 (segment (start 48.514 38.0365) (end 48.9585 38.481) (width 0.254) (layer F.Cu) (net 2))
 (segment (start 41.1607 26.1874) (end 41.1607 26.9113) (width 0.254) (layer F.Cu) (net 4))
 (segment (start 40.9956 31.242) (end 42.418 31.242) (width 0.254) (layer F.Cu) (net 4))
 (segment (start 40.64 30.8864) (end 40.9956 31.242) (width 0.254) (layer F.Cu) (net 4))
 (segment (start 40.64 27.432) (end 40.64 30.8864) (width 0.254) (layer F.Cu) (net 4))
 (segment (start 41.1607 26.9113) (end 40.64 27.432) (width 0.254) (layer F.Cu) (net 4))
 (segment (start 42.418 31.242) (end 43.815 31.242) (width 0.254) (layer F.Cu) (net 4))
 (segment (start 43.815 31.242) (end 44.831 32.258) (width 0.254) (layer F.Cu) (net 4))
 (segment (start 44.831 32.258) (end 45.9105 32.258) (width 0.254) (layer F.Cu) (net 4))
 (segment (start 45.9105 32.258) (end 46.0375 32.131) (width 0.254) (layer F.Cu) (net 4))
 (segment (start 41.1607 23.6474) (end 41.1607 26.1874) (width 0.254) (layer F.Cu) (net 4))
 (segment (start 42.799 22.2504) (end 42.799 21.463) (width 0.254) (layer F.Cu) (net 5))
 (segment (start 42.6974 21.3614) (end 41.1607 21.3614) (width 0.254) (layer F.Cu) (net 5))
 (segment (start 42.799 21.463) (end 42.6974 21.3614) (width 0.254) (layer F.Cu) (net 5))
 (segment (start 42.418 29.972) (end 41.275 29.972) (width 0.254) (layer F.Cu) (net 5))
 (segment (start 41.275 27.94) (end 43.053 26.162) (width 0.254) (layer F.Cu) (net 5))
 (segment (start 41.275 29.972) (end 41.275 27.94) (width 0.254) (layer F.Cu) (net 5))
 (segment (start 42.799 22.987) (end 42.799 25.908) (width 0.254) (layer F.Cu) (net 5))
 (segment (start 43.30192 26.28392) (end 45.085 26.28392) (width 0.254) (layer F.Cu) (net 5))
 (segment (start 43.17492 26.28392) (end 43.30192 26.28392) (width 0.254) (layer F.Cu) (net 5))
 (segment (start 42.799 25.908) (end 43.053 26.162) (width 0.254) (layer F.Cu) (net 5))
 (segment (start 43.053 26.162) (end 43.17492 26.28392) (width 0.254) (layer F.Cu) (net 5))
 (segment (start 46.2915 28.575) (end 46.2915 28.2575) (width 0.254) (layer F.Cu) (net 5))
 (segment (start 47.498 27.051) (end 47.498 26.28392) (width 0.254) (layer F.Cu) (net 5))
 (segment (start 46.2915 28.2575) (end 47.498 27.051) (width 0.254) (layer F.Cu) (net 5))
 (segment (start 42.799 23.114) (end 42.799 22.987) (width 0.254) (layer F.Cu) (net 5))
 (segment (start 42.799 22.987) (end 42.799 22.2504) (width 0.254) (layer F.Cu) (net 5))
 (segment (start 42.799 22.2504) (end 42.799 21.971) (width 0.254) (layer F.Cu) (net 5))
 (segment (start 42.799 22.733) (end 42.799 23.114) (width 0.254) (layer F.Cu) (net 5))
 (segment (start 44.831 26.28392) (end 47.498 26.28392) (width 0.254) (layer F.Cu) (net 5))
 (segment (start 47.498 26.28392) (end 49.657 26.28392) (width 0.254) (layer F.Cu) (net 5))
 (segment (start 44.831 26.28392) (end 44.831 27.1145) (width 0.254) (layer F.Cu) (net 5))
 (segment (start 44.831 27.1145) (end 46.2915 28.575) (width 0.254) (layer F.Cu) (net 5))
 (segment (start 44.20108 26.28392) (end 44.831 26.28392) (width 0.254) (layer F.Cu) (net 5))
 (segment (start 46.0629 19.939) (end 53.5432 19.939) (width 0.254) (layer F.Cu) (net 6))
 (segment (start 53.975 21.209) (end 53.975 27.686) (width 0.254) (layer F.Cu) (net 6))
 (segment (start 53.975 21.082) (end 53.975 21.209) (width 0.254) (layer F.Cu) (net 6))
 (segment (start 53.975 20.3708) (end 53.975 21.082) (width 0.254) (layer F.Cu) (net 6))
 (segment (start 53.5432 19.939) (end 53.975 20.3708) (width 0.254) (layer F.Cu) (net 6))
 (segment (start 52.7685 32.385) (end 52.7685 30.6705) (width 0.254) (layer F.Cu) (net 6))
 (segment (start 52.7685 30.6705) (end 52.6415 30.5435) (width 0.254) (layer F.Cu) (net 6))
 (segment (start 42.418 28.702) (end 44.2595 28.702) (width 0.254) (layer F.Cu) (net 6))
 (segment (start 44.2595 28.702) (end 44.3865 28.575) (width 0.254) (layer F.Cu) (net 6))
 (segment (start 48.3235 30.5435) (end 52.6415 30.5435) (width 0.254) (layer F.Cu) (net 6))
 (segment (start 52.6415 30.5435) (end 52.7685 30.5435) (width 0.254) (layer F.Cu) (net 6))
 (segment (start 52.7685 30.5435) (end 52.7685 28.8925) (width 0.254) (layer F.Cu) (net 6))
 (segment (start 52.7685 28.8925) (end 53.086 28.575) (width 0.254) (layer F.Cu) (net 6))
 (segment (start 53.086 28.575) (end 53.721 28.575) (width 0.254) (layer F.Cu) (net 6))
 (segment (start 53.975 28.321) (end 53.975 27.813) (width 0.254) (layer F.Cu) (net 6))
 (segment (start 53.721 28.575) (end 53.975 28.321) (width 0.254) (layer F.Cu) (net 6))
 (segment (start 44.3865 28.575) (end 44.3865 30.0355) (width 0.254) (layer F.Cu) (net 6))
 (segment (start 48.4505 30.4165) (end 48.4505 29.21) (width 0.254) (layer F.Cu) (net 6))
 (segment (start 48.133 30.734) (end 48.3235 30.5435) (width 0.254) (layer F.Cu) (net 6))
 (segment (start 48.3235 30.5435) (end 48.4505 30.4165) (width 0.254) (layer F.Cu) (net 6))
 (segment (start 45.085 30.734) (end 48.133 30.734) (width 0.254) (layer F.Cu) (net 6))
 (segment (start 44.3865 30.0355) (end 45.085 30.734) (width 0.254) (layer F.Cu) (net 6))
 (segment (start 44.1325 28.321) (end 44.3865 28.575) (width 0.254) (layer F.Cu) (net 6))
 (segment (start 40.0558 19.939) (end 40.0558 17.3282) (width 0.254) (layer F.Cu) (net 9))
 (segment (start 40.0558 17.3282) (end 39.8726 17.145) (width 0.254) (layer F.Cu) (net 9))
 (segment (start 35.5473 21.4376) (end 35.5473 20.1803) (width 0.254) (layer F.Cu) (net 9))
 (segment (start 35.7886 19.939) (end 40.0558 19.939) (width 0.254) (layer F.Cu) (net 9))
 (segment (start 40.0558 19.939) (end 44.1579 19.939) (width 0.254) (layer F.Cu) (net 9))
 (segment (start 35.5473 20.1803) (end 35.7886 19.939) (width 0.254) (layer F.Cu) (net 9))
 (segment (start 35.5473 21.4376) (end 33.909 21.4376) (width 0.254) (layer F.Cu) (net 9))
 (segment (start 36.5252 25.4508) (end 36.5252 22.6568) (width 0.254) (layer F.Cu) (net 9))
 (segment (start 35.5473 21.6789) (end 35.5473 21.4376) (width 0.254) (layer F.Cu) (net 9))
 (segment (start 36.5252 22.6568) (end 35.5473 21.6789) (width 0.254) (layer F.Cu) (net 9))
 (segment (start 36.83 31.242) (end 38.608 31.242) (width 0.254) (layer F.Cu) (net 9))
 (segment (start 36.5252 27.0256) (end 36.5252 25.4508) (width 0.254) (layer F.Cu) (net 9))
 (segment (start 36.5252 25.4508) (end 36.5252 25.0952) (width 0.254) (layer F.Cu) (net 9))
 (segment (start 36.7284 27.2288) (end 36.5252 27.0256) (width 0.254) (layer F.Cu) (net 9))
 (segment (start 38.1508 27.2288) (end 36.7284 27.2288) (width 0.254) (layer F.Cu) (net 9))
 (segment (start 38.6588 27.7368) (end 38.1508 27.2288) (width 0.254) (layer F.Cu) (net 9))
 (segment (start 38.6588 31.1912) (end 38.6588 27.7368) (width 0.254) (layer F.Cu) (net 9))
 (segment (start 38.608 31.242) (end 38.6588 31.1912) (width 0.254) (layer F.Cu) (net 9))
 (segment (start 42.829 44.3122) (end 42.829 45.521398) (width 0.254) (layer F.Cu) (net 10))
 (segment (start 50.6135 45.589) (end 50.6135 44.3865) (width 0.254) (layer F.Cu) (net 10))
 (segment (start 50.6135 44.3865) (end 50.6135 38.604) (width 0.254) (layer F.Cu) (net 10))
 (segment (start 50.6135 38.604) (end 50.7365 38.481) (width 0.254) (layer F.Cu) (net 10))
 (segment (start 50.3555 45.847) (end 50.6135 45.589) (width 0.254) (layer F.Cu) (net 10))
 (segment (start 43.154602 45.847) (end 50.3555 45.847) (width 0.254) (layer F.Cu) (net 10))
 (segment (start 42.829 45.521398) (end 43.154602 45.847) (width 0.254) (layer F.Cu) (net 10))
 (segment (start 43.1292 37.1348) (end 43.8023 37.1348) (width 0.254) (layer F.Cu) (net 10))
 (segment (start 43.8023 37.1348) (end 43.9674 37.2999) (width 0.254) (layer F.Cu) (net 10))
 (segment (start 43.9674 37.2999) (end 43.9674 43.18) (width 0.254) (layer F.Cu) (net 10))
 (segment (start 43.9674 43.18) (end 42.8352 44.3122) (width 0.254) (layer F.Cu) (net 10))
 (segment (start 42.8352 44.3122) (end 42.829 44.3122) (width 0.254) (layer F.Cu) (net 10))
 (segment (start 41.1607 37.1348) (end 43.1292 37.1348) (width 0.254) (layer F.Cu) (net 10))
 (segment (start 50.8 36.3855) (end 48.5775 36.3855) (width 0.254) (layer F.Cu) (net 10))
 (segment (start 48.5775 36.3855) (end 48.514 36.322) (width 0.254) (layer F.Cu) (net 10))
 (segment (start 50.7365 38.481) (end 50.7365 36.449) (width 0.254) (layer F.Cu) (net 10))
 (segment (start 50.7365 36.449) (end 50.8 36.3855) (width 0.254) (layer F.Cu) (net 10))
 (segment (start 38.6715 32.512) (end 39.751 33.3375) (width 0.254) (layer F.Cu) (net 10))
 (segment (start 39.751 33.3375) (end 39.751 36.2585) (width 0.254) (layer F.Cu) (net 10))
 (segment (start 39.751 36.2585) (end 41.1607 37.1348) (width 0.254) (layer F.Cu) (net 10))
 (segment (start 41.1607 37.1348) (end 41.0972 37.0713) (width 0.254) (layer F.Cu) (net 10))
 (segment (start 36.83 32.512) (end 38.6715 32.512) (width 0.254) (layer F.Cu) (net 10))
 (segment (start 38.9636 36.4617) (end 38.9636 36.6649) (width 0.254) (layer F.Cu) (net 7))
 (segment (start 37.7298 44.3122) (end 37.729 44.3122) (width 0.254) (layer F.Cu) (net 7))
 (segment (start 39.4589 42.5831) (end 37.7298 44.3122) (width 0.254) (layer F.Cu) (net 7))
 (segment (start 39.4589 37.1602) (end 39.4589 42.5831) (width 0.254) (layer F.Cu) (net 7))
 (segment (start 38.9636 36.6649) (end 39.4589 37.1602) (width 0.254) (layer F.Cu) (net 7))
 (segment (start 38.6334 33.782) (end 36.83 33.782) (width 0.254) (layer F.Cu) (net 7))
 (segment (start 38.9636 34.1122) (end 38.6334 33.782) (width 0.254) (layer F.Cu) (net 7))
 (segment (start 38.9636 36.5252) (end 38.9636 36.4617) (width 0.254) (layer F.Cu) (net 7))
 (segment (start 38.9636 36.4617) (end 38.9636 34.1122) (width 0.254) (layer F.Cu) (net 7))
 (segment (start 34.8615 32.004) (end 34.8615 33.4137) (width 0.254) (layer F.Cu) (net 7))
 (segment (start 35.2298 33.782) (end 36.83 33.782) (width 0.254) (layer F.Cu) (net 7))
 (segment (start 34.8615 33.4137) (end 35.2298 33.782) (width 0.254) (layer F.Cu) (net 7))
 (segment (start 36.83 28.702) (end 35.4584 28.702) (width 0.254) (layer F.Cu) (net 7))
 (segment (start 35.4584 28.702) (end 34.8615 29.2989) (width 0.254) (layer F.Cu) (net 7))
 (segment (start 34.8615 29.2989) (end 34.8615 32.004) (width 0.254) (layer F.Cu) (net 7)))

